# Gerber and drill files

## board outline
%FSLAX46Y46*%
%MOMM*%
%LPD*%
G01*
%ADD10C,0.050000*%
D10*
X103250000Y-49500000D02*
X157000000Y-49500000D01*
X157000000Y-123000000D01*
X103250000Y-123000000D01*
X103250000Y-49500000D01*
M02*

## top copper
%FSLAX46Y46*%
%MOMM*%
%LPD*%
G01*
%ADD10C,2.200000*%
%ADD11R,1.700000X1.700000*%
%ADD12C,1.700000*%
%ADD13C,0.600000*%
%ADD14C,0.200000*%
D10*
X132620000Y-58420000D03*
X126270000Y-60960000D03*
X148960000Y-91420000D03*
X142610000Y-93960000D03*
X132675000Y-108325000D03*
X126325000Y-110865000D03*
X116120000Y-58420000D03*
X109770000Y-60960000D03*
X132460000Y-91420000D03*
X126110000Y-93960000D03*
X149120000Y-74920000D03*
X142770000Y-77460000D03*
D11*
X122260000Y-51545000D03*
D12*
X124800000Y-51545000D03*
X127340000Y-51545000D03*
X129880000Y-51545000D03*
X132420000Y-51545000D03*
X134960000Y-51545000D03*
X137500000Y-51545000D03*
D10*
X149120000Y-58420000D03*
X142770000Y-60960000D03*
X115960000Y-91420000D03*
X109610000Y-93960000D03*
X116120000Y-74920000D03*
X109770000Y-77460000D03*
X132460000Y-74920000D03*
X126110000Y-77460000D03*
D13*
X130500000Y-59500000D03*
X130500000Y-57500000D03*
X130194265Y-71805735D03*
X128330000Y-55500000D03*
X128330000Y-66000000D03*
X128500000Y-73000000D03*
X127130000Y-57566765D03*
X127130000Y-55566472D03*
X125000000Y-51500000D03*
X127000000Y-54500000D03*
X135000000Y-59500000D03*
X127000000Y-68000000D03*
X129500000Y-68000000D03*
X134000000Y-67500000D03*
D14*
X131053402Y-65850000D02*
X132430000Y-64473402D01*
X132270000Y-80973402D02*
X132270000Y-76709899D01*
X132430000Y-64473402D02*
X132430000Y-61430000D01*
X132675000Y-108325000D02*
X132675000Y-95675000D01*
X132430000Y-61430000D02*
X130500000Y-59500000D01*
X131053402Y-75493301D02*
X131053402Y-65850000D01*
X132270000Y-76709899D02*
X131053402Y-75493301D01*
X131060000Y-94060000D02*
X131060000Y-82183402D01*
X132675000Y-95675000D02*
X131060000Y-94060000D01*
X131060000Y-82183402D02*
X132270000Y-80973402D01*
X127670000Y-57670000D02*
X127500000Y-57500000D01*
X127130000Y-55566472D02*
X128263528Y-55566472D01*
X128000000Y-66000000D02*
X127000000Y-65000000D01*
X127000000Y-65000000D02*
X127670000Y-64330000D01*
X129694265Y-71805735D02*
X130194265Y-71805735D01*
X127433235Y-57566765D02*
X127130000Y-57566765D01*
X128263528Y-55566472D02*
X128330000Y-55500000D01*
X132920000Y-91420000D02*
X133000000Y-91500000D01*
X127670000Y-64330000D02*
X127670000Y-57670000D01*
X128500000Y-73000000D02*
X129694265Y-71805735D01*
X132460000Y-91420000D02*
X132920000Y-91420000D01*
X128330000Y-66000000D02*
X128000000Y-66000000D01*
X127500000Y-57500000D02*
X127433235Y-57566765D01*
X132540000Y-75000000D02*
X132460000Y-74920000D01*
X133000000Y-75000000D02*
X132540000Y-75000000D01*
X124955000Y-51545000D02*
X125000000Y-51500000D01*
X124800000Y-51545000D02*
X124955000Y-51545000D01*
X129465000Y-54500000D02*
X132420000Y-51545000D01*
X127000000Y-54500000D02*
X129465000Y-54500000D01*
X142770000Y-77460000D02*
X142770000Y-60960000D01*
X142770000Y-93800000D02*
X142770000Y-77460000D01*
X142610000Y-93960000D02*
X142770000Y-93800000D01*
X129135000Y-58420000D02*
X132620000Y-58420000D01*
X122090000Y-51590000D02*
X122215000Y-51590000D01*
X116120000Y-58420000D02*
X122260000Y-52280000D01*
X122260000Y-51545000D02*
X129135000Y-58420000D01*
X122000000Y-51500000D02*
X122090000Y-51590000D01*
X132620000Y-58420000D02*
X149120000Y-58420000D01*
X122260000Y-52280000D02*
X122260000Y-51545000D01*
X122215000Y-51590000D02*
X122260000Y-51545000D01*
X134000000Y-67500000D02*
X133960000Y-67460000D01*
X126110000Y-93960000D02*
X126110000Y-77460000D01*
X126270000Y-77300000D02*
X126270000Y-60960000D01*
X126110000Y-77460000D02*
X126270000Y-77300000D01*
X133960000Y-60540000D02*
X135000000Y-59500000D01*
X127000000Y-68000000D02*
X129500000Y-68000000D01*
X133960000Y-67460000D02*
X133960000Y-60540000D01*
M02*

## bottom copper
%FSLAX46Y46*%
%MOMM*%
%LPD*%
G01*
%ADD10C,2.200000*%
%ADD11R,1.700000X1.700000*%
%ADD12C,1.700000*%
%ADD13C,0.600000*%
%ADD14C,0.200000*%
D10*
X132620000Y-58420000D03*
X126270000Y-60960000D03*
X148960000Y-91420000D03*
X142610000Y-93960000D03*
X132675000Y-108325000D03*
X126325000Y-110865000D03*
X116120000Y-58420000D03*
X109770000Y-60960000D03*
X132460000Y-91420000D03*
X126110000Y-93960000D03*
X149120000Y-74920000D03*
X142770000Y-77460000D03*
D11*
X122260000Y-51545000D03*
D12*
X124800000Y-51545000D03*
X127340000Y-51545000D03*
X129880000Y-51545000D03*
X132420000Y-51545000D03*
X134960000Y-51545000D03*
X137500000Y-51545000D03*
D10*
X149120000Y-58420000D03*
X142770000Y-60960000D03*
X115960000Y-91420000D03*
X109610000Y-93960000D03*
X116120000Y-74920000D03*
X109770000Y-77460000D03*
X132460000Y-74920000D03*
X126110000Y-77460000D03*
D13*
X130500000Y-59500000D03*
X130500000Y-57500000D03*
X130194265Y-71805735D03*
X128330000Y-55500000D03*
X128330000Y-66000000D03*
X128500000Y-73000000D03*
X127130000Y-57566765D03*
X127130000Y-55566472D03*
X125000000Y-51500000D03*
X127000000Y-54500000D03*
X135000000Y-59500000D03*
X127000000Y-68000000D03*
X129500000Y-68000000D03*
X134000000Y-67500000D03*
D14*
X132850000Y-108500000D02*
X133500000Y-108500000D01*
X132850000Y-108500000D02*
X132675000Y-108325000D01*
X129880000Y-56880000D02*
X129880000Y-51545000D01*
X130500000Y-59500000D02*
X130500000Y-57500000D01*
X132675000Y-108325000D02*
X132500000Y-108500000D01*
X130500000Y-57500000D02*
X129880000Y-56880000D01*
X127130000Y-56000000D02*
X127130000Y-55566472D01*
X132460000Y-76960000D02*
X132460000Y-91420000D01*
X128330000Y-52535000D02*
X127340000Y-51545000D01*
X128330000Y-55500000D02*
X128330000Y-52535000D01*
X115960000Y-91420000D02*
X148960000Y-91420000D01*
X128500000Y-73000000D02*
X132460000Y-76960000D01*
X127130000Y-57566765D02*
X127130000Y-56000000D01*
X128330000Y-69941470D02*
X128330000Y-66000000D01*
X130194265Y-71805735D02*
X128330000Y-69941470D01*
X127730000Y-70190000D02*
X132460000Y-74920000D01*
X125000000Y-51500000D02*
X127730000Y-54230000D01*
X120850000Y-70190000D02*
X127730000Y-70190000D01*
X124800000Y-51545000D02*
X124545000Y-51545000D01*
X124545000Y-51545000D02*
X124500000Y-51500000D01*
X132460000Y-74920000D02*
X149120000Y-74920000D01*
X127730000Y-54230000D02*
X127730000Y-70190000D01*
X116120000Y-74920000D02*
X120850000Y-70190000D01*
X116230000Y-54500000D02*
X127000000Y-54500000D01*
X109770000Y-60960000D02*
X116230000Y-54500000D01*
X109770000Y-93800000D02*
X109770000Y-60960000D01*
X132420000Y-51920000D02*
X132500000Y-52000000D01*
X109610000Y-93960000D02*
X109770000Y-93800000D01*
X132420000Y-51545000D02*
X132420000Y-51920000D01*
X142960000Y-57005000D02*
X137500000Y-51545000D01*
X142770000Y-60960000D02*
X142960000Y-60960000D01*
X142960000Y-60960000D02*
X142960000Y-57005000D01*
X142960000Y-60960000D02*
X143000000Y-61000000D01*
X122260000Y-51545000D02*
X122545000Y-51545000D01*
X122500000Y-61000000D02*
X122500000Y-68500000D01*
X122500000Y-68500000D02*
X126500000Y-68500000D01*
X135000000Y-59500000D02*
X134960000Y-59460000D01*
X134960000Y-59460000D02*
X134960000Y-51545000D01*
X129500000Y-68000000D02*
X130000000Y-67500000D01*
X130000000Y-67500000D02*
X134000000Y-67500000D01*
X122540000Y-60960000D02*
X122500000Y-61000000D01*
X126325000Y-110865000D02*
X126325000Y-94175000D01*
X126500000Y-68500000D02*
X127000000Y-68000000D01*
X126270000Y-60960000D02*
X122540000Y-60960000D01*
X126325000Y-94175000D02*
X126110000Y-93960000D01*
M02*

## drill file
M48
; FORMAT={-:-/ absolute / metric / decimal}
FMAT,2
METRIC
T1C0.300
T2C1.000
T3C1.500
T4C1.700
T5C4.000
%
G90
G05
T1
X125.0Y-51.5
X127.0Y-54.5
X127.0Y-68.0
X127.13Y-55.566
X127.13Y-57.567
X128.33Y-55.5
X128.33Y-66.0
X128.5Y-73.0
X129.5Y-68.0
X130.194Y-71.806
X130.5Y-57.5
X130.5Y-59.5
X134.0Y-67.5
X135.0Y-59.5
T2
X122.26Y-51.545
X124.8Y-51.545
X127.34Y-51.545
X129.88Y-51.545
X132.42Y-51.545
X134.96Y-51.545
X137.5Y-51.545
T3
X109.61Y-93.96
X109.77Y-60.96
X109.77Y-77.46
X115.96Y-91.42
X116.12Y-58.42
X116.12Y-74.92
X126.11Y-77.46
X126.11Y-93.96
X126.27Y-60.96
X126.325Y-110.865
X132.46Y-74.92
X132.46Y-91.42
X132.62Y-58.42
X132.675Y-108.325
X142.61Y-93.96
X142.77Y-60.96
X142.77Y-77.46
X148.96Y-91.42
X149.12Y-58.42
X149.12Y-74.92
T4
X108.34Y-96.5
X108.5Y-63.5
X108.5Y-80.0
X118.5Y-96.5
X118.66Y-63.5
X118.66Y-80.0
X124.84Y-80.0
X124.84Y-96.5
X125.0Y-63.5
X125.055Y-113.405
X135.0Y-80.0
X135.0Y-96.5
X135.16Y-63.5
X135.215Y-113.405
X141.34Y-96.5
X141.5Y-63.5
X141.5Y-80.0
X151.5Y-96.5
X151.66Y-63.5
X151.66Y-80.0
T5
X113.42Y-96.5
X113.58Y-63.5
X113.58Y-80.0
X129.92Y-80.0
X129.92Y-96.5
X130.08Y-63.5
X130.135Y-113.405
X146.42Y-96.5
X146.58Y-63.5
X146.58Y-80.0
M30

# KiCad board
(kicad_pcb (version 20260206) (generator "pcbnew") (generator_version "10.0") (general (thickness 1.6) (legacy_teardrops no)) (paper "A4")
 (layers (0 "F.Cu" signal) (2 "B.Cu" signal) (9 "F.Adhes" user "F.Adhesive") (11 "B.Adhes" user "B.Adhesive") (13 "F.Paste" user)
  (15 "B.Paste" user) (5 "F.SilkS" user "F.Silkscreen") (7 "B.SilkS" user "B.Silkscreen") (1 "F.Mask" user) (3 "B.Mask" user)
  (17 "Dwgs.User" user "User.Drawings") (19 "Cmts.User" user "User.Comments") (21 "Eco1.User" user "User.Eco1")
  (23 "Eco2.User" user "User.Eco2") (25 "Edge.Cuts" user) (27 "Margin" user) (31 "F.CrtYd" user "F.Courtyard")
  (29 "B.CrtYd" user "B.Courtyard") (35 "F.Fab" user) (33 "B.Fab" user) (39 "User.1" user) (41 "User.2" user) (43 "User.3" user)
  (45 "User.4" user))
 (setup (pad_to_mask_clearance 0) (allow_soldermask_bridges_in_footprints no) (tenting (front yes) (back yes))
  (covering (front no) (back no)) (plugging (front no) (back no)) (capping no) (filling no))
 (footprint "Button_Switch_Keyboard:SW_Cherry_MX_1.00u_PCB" (layer "F.Cu") (at 132.62 58.42)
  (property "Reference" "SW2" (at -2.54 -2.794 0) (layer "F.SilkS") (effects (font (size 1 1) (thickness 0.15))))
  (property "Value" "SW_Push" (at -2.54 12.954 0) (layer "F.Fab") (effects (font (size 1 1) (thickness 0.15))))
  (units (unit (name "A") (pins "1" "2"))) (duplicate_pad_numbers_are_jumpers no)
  (pad "" np_thru_hole circle (at -7.62 5.08) (size 1.7 1.7) (drill 1.7) (layers "*.Cu" "*.Mask"))
  (pad "" np_thru_hole circle (at -2.54 5.08) (size 4 4) (drill 4) (layers "*.Cu" "*.Mask"))
  (pad "" np_thru_hole circle (at 2.54 5.08) (size 1.7 1.7) (drill 1.7) (layers "*.Cu" "*.Mask"))
  (pad "1" thru_hole circle (at 0 0) (size 2.2 2.2) (drill 1.5) (layers "*.Cu" "*.Mask") (remove_unused_layers no) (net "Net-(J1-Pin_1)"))
  (pad "2" thru_hole circle (at -6.35 2.54) (size 2.2 2.2) (drill 1.5) (layers "*.Cu" "*.Mask") (remove_unused_layers no)
   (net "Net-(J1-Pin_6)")))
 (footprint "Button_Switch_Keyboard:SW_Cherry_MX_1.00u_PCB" (layer "F.Cu") (at 148.96 91.42)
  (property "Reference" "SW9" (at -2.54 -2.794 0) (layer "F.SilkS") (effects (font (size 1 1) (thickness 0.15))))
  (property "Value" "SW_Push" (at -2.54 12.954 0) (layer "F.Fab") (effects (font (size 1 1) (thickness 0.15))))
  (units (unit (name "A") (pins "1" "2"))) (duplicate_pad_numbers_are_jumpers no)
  (pad "" np_thru_hole circle (at -7.62 5.08) (size 1.7 1.7) (drill 1.7) (layers "*.Cu" "*.Mask"))
  (pad "" np_thru_hole circle (at -2.54 5.08) (size 4 4) (drill 4) (layers "*.Cu" "*.Mask"))
  (pad "" np_thru_hole circle (at 2.54 5.08) (size 1.7 1.7) (drill 1.7) (layers "*.Cu" "*.Mask"))
  (pad "1" thru_hole circle (at 0 0) (size 2.2 2.2) (drill 1.5) (layers "*.Cu" "*.Mask") (remove_unused_layers no) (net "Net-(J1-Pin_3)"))
  (pad "2" thru_hole circle (at -6.35 2.54) (size 2.2 2.2) (drill 1.5) (layers "*.Cu" "*.Mask") (remove_unused_layers no)
   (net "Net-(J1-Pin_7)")))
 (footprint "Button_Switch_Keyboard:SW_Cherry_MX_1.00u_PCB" (layer "F.Cu") (at 132.675 108.325)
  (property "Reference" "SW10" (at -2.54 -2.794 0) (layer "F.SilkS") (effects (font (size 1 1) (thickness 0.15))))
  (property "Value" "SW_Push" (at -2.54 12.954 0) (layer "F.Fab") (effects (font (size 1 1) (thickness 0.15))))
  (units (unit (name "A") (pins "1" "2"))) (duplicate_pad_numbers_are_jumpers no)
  (pad "" np_thru_hole circle (at -7.62 5.08) (size 1.7 1.7) (drill 1.7) (layers "*.Cu" "*.Mask"))
  (pad "" np_thru_hole circle (at -2.54 5.08) (size 4 4) (drill 4) (layers "*.Cu" "*.Mask"))
  (pad "" np_thru_hole circle (at 2.54 5.08) (size 1.7 1.7) (drill 1.7) (layers "*.Cu" "*.Mask"))
  (pad "1" thru_hole circle (at 0 0) (size 2.2 2.2) (drill 1.5) (layers "*.Cu" "*.Mask") (remove_unused_layers no) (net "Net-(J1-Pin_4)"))
  (pad "2" thru_hole circle (at -6.35 2.54) (size 2.2 2.2) (drill 1.5) (layers "*.Cu" "*.Mask") (remove_unused_layers no)
   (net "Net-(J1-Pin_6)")))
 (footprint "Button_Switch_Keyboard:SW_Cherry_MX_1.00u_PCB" (layer "F.Cu") (at 116.12 58.42)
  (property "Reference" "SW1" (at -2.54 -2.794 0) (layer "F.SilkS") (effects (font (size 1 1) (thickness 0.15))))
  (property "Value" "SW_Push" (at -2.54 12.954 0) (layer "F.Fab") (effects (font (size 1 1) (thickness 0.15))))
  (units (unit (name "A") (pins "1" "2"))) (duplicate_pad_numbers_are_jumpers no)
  (pad "" np_thru_hole circle (at -7.62 5.08) (size 1.7 1.7) (drill 1.7) (layers "*.Cu" "*.Mask"))
  (pad "" np_thru_hole circle (at -2.54 5.08) (size 4 4) (drill 4) (layers "*.Cu" "*.Mask"))
  (pad "" np_thru_hole circle (at 2.54 5.08) (size 1.7 1.7) (drill 1.7) (layers "*.Cu" "*.Mask"))
  (pad "1" thru_hole circle (at 0 0) (size 2.2 2.2) (drill 1.5) (layers "*.Cu" "*.Mask") (remove_unused_layers no) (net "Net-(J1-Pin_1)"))
  (pad "2" thru_hole circle (at -6.35 2.54) (size 2.2 2.2) (drill 1.5) (layers "*.Cu" "*.Mask") (remove_unused_layers no)
   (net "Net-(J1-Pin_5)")))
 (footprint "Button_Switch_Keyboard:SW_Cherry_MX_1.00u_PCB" (layer "F.Cu") (at 132.46 91.42)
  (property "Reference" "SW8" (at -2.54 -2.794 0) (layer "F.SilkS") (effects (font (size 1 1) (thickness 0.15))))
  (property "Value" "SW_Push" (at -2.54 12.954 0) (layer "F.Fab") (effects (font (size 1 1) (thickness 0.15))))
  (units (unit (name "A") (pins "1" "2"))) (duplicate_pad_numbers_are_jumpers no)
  (pad "" np_thru_hole circle (at -7.62 5.08) (size 1.7 1.7) (drill 1.7) (layers "*.Cu" "*.Mask"))
  (pad "" np_thru_hole circle (at -2.54 5.08) (size 4 4) (drill 4) (layers "*.Cu" "*.Mask"))
  (pad "" np_thru_hole circle (at 2.54 5.08) (size 1.7 1.7) (drill 1.7) (layers "*.Cu" "*.Mask"))
  (pad "1" thru_hole circle (at 0 0) (size 2.2 2.2) (drill 1.5) (layers "*.Cu" "*.Mask") (remove_unused_layers no) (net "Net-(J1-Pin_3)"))
  (pad "2" thru_hole circle (at -6.35 2.54) (size 2.2 2.2) (drill 1.5) (layers "*.Cu" "*.Mask") (remove_unused_layers no)
   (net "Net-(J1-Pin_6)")))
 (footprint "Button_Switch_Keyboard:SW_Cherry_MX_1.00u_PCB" (layer "F.Cu") (at 149.12 74.92)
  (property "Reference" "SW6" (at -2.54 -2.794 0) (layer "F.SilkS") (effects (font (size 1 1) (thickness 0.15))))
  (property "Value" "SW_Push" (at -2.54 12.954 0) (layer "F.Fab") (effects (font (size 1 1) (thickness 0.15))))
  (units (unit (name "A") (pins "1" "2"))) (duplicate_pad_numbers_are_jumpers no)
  (pad "" np_thru_hole circle (at -7.62 5.08) (size 1.7 1.7) (drill 1.7) (layers "*.Cu" "*.Mask"))
  (pad "" np_thru_hole circle (at -2.54 5.08) (size 4 4) (drill 4) (layers "*.Cu" "*.Mask"))
  (pad "" np_thru_hole circle (at 2.54 5.08) (size 1.7 1.7) (drill 1.7) (layers "*.Cu" "*.Mask"))
  (pad "1" thru_hole circle (at 0 0) (size 2.2 2.2) (drill 1.5) (layers "*.Cu" "*.Mask") (remove_unused_layers no) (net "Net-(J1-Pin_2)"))
  (pad "2" thru_hole circle (at -6.35 2.54) (size 2.2 2.2) (drill 1.5) (layers "*.Cu" "*.Mask") (remove_unused_layers no)
   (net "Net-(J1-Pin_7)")))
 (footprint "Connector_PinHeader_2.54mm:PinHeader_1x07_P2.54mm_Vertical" (layer "F.Cu") (at 122.26 51.545 90)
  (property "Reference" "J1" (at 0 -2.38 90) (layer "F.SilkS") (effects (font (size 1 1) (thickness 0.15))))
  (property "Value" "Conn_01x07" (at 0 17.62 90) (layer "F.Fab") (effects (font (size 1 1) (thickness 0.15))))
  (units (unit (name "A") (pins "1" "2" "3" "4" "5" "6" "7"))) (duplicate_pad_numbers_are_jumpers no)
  (pad "1" thru_hole rect (at 0 0 90) (size 1.7 1.7) (drill 1) (layers "*.Cu" "*.Mask") (remove_unused_layers no) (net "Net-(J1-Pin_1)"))
  (pad "2" thru_hole circle (at 0 2.54 90) (size 1.7 1.7) (drill 1) (layers "*.Cu" "*.Mask") (remove_unused_layers no)
   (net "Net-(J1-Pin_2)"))
  (pad "3" thru_hole circle (at 0 5.08 90) (size 1.7 1.7) (drill 1) (layers "*.Cu" "*.Mask") (remove_unused_layers no)
   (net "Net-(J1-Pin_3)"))
  (pad "4" thru_hole circle (at 0 7.62 90) (size 1.7 1.7) (drill 1) (layers "*.Cu" "*.Mask") (remove_unused_layers no)
   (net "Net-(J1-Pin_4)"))
  (pad "5" thru_hole circle (at 0 10.16 90) (size 1.7 1.7) (drill 1) (layers "*.Cu" "*.Mask") (remove_unused_layers no)
   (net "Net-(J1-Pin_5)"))
  (pad "6" thru_hole circle (at 0 12.7 90) (size 1.7 1.7) (drill 1) (layers "*.Cu" "*.Mask") (remove_unused_layers no)
   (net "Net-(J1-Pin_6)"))
  (pad "7" thru_hole circle (at 0 15.24 90) (size 1.7 1.7) (drill 1) (layers "*.Cu" "*.Mask") (remove_unused_layers no)
   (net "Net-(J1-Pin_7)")))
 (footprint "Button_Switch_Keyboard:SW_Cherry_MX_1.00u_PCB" (layer "F.Cu") (at 149.12 58.42)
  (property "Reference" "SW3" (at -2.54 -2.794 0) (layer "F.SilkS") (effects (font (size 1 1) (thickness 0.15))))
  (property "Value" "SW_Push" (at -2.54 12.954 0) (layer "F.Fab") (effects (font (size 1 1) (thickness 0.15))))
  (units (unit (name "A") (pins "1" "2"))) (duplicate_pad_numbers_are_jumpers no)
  (pad "" np_thru_hole circle (at -7.62 5.08) (size 1.7 1.7) (drill 1.7) (layers "*.Cu" "*.Mask"))
  (pad "" np_thru_hole circle (at -2.54 5.08) (size 4 4) (drill 4) (layers "*.Cu" "*.Mask"))
  (pad "" np_thru_hole circle (at 2.54 5.08) (size 1.7 1.7) (drill 1.7) (layers "*.Cu" "*.Mask"))
  (pad "1" thru_hole circle (at 0 0) (size 2.2 2.2) (drill 1.5) (layers "*.Cu" "*.Mask") (remove_unused_layers no) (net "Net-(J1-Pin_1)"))
  (pad "2" thru_hole circle (at -6.35 2.54) (size 2.2 2.2) (drill 1.5) (layers "*.Cu" "*.Mask") (remove_unused_layers no)
   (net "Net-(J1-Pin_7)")))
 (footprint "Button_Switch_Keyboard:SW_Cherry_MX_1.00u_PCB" (layer "F.Cu") (at 115.96 91.42)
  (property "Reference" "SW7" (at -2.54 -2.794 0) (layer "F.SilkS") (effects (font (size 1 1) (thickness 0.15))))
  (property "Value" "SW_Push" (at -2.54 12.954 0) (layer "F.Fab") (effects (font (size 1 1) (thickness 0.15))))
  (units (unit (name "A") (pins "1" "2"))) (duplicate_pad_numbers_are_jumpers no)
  (pad "" np_thru_hole circle (at -7.62 5.08) (size 1.7 1.7) (drill 1.7) (layers "*.Cu" "*.Mask"))
  (pad "" np_thru_hole circle (at -2.54 5.08) (size 4 4) (drill 4) (layers "*.Cu" "*.Mask"))
  (pad "" np_thru_hole circle (at 2.54 5.08) (size 1.7 1.7) (drill 1.7) (layers "*.Cu" "*.Mask"))
  (pad "1" thru_hole circle (at 0 0) (size 2.2 2.2) (drill 1.5) (layers "*.Cu" "*.Mask") (remove_unused_layers no) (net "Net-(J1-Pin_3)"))
  (pad "2" thru_hole circle (at -6.35 2.54) (size 2.2 2.2) (drill 1.5) (layers "*.Cu" "*.Mask") (remove_unused_layers no)
   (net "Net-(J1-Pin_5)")))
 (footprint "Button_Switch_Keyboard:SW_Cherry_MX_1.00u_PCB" (layer "F.Cu") (at 116.12 74.92)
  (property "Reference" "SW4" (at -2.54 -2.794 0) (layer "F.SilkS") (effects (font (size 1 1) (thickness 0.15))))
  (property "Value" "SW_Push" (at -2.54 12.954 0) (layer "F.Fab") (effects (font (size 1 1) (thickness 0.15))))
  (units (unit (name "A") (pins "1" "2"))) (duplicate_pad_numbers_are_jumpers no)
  (pad "" np_thru_hole circle (at -7.62 5.08) (size 1.7 1.7) (drill 1.7) (layers "*.Cu" "*.Mask"))
  (pad "" np_thru_hole circle (at -2.54 5.08) (size 4 4) (drill 4) (layers "*.Cu" "*.Mask"))
  (pad "" np_thru_hole circle (at 2.54 5.08) (size 1.7 1.7) (drill 1.7) (layers "*.Cu" "*.Mask"))
  (pad "1" thru_hole circle (at 0 0) (size 2.2 2.2) (drill 1.5) (layers "*.Cu" "*.Mask") (remove_unused_layers no) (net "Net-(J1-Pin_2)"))
  (pad "2" thru_hole circle (at -6.35 2.54) (size 2.2 2.2) (drill 1.5) (layers "*.Cu" "*.Mask") (remove_unused_layers no)
   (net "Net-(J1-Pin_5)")))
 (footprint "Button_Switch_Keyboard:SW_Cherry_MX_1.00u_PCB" (layer "F.Cu") (at 132.46 74.92)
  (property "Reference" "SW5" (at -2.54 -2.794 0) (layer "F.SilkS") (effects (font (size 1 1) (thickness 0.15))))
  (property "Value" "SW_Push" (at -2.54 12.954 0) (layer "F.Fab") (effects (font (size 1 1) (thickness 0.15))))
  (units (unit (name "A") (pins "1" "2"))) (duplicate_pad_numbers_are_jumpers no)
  (pad "" np_thru_hole circle (at -7.62 5.08) (size 1.7 1.7) (drill 1.7) (layers "*.Cu" "*.Mask"))
  (pad "" np_thru_hole circle (at -2.54 5.08) (size 4 4) (drill 4) (layers "*.Cu" "*.Mask"))
  (pad "" np_thru_hole circle (at 2.54 5.08) (size 1.7 1.7) (drill 1.7) (layers "*.Cu" "*.Mask"))
  (pad "1" thru_hole circle (at 0 0) (size 2.2 2.2) (drill 1.5) (layers "*.Cu" "*.Mask") (remove_unused_layers no) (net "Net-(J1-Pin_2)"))
  (pad "2" thru_hole circle (at -6.35 2.54) (size 2.2 2.2) (drill 1.5) (layers "*.Cu" "*.Mask") (remove_unused_layers no)
   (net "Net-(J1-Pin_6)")))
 (gr_rect (start 103.25 49.5) (end 157 123) (stroke (width 0.05) (type default)) (fill no) (layer "Edge.Cuts"))
 (segment (start 131.053402 65.85) (end 132.43 64.473402) (width 0.2) (layer "F.Cu") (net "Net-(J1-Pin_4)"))
 (segment (start 132.27 80.973402) (end 132.27 76.709899) (width 0.2) (layer "F.Cu") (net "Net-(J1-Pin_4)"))
 (segment (start 132.43 64.473402) (end 132.43 61.43) (width 0.2) (layer "F.Cu") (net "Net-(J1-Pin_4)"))
 (segment (start 132.675 108.325) (end 132.675 95.675) (width 0.2) (layer "F.Cu") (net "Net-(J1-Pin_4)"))
 (segment (start 132.43 61.43) (end 130.5 59.5) (width 0.2) (layer "F.Cu") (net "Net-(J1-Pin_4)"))
 (segment (start 131.053402 75.493301) (end 131.053402 65.85) (width 0.2) (layer "F.Cu") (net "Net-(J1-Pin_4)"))
 (segment (start 132.27 76.709899) (end 131.053402 75.493301) (width 0.2) (layer "F.Cu") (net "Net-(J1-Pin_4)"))
 (segment (start 131.06 94.06) (end 131.06 82.183402) (width 0.2) (layer "F.Cu") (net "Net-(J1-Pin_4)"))
 (segment (start 132.675 95.675) (end 131.06 94.06) (width 0.2) (layer "F.Cu") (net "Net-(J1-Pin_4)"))
 (segment (start 131.06 82.183402) (end 132.27 80.973402) (width 0.2) (layer "F.Cu") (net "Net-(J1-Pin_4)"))
 (via (at 130.5 59.5) (size 0.6) (drill 0.3) (layers "F.Cu" "B.Cu") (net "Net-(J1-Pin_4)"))
 (via (at 130.5 57.5) (size 0.6) (drill 0.3) (layers "F.Cu" "B.Cu") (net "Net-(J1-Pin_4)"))
 (segment (start 132.85 108.5) (end 133.5 108.5) (width 0.2) (layer "B.Cu") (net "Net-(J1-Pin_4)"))
 (segment (start 132.85 108.5) (end 132.675 108.325) (width 0.2) (layer "B.Cu") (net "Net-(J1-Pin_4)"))
 (segment (start 129.88 56.88) (end 129.88 51.545) (width 0.2) (layer "B.Cu") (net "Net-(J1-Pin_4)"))
 (segment (start 130.5 59.5) (end 130.5 57.5) (width 0.2) (layer "B.Cu") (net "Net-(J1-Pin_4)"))
 (segment (start 132.675 108.325) (end 132.5 108.5) (width 0.2) (layer "B.Cu") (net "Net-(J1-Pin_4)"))
 (segment (start 130.5 57.5) (end 129.88 56.88) (width 0.2) (layer "B.Cu") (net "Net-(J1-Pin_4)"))
 (segment (start 127.67 57.67) (end 127.5 57.5) (width 0.2) (layer "F.Cu") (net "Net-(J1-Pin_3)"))
 (segment (start 127.13 55.566472) (end 128.263528 55.566472) (width 0.2) (layer "F.Cu") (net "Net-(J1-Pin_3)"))
 (segment (start 128 66) (end 127 65) (width 0.2) (layer "F.Cu") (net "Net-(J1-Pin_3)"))
 (segment (start 127 65) (end 127.67 64.33) (width 0.2) (layer "F.Cu") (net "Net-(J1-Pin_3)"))
 (segment (start 129.694265 71.805735) (end 130.194265 71.805735) (width 0.2) (layer "F.Cu") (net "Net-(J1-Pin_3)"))
 (segment (start 127.433235 57.566765) (end 127.13 57.566765) (width 0.2) (layer "F.Cu") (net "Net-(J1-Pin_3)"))
 (segment (start 128.263528 55.566472) (end 128.33 55.5) (width 0.2) (layer "F.Cu") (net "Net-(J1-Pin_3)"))
 (segment (start 132.92 91.42) (end 133 91.5) (width 0.2) (layer "F.Cu") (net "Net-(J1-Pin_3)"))
 (segment (start 127.67 64.33) (end 127.67 57.67) (width 0.2) (layer "F.Cu") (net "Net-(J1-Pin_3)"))
 (segment (start 128.5 73) (end 129.694265 71.805735) (width 0.2) (layer "F.Cu") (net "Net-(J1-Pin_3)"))
 (segment (start 132.46 91.42) (end 132.92 91.42) (width 0.2) (layer "F.Cu") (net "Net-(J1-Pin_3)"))
 (segment (start 128.33 66) (end 128 66) (width 0.2) (layer "F.Cu") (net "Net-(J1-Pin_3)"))
 (segment (start 127.5 57.5) (end 127.433235 57.566765) (width 0.2) (layer "F.Cu") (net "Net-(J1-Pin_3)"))
 (via (at 130.194265 71.805735) (size 0.6) (drill 0.3) (layers "F.Cu" "B.Cu") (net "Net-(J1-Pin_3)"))
 (via (at 128.33 55.5) (size 0.6) (drill 0.3) (layers "F.Cu" "B.Cu") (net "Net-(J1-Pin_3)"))
 (via (at 128.33 66) (size 0.6) (drill 0.3) (layers "F.Cu" "B.Cu") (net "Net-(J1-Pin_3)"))
 (via (at 128.5 73) (size 0.6) (drill 0.3) (layers "F.Cu" "B.Cu") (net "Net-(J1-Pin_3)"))
 (via (at 127.13 57.566765) (size 0.6) (drill 0.3) (layers "F.Cu" "B.Cu") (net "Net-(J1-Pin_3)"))
 (via (at 127.13 55.566472) (size 0.6) (drill 0.3) (layers "F.Cu" "B.Cu") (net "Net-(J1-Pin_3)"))
 (segment (start 127.13 56) (end 127.13 55.566472) (width 0.2) (layer "B.Cu") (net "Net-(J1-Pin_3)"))
 (segment (start 132.46 76.96) (end 132.46 91.42) (width 0.2) (layer "B.Cu") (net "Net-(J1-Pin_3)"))
 (segment (start 128.33 52.535) (end 127.34 51.545) (width 0.2) (layer "B.Cu") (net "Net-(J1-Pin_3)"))
 (segment (start 128.33 55.5) (end 128.33 52.535) (width 0.2) (layer "B.Cu") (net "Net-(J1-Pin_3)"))
 (segment (start 115.96 91.42) (end 148.96 91.42) (width 0.2) (layer "B.Cu") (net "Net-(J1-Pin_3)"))
 (segment (start 128.5 73) (end 132.46 76.96) (width 0.2) (layer "B.Cu") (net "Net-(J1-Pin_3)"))
 (segment (start 127.13 57.566765) (end 127.13 56) (width 0.2) (layer "B.Cu") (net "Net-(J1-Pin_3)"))
 (segment (start 128.33 69.94147) (end 128.33 66) (width 0.2) (layer "B.Cu") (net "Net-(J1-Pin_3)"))
 (segment (start 130.194265 71.805735) (end 128.33 69.94147) (width 0.2) (layer "B.Cu") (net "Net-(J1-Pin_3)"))
 (segment (start 132.54 75) (end 132.46 74.92) (width 0.2) (layer "F.Cu") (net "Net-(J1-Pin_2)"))
 (segment (start 133 75) (end 132.54 75) (width 0.2) (layer "F.Cu") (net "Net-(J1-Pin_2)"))
 (segment (start 124.955 51.545) (end 125 51.5) (width 0.2) (layer "F.Cu") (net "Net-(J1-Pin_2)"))
 (segment (start 124.8 51.545) (end 124.955 51.545) (width 0.2) (layer "F.Cu") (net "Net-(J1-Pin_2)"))
 (via (at 125 51.5) (size 0.6) (drill 0.3) (layers "F.Cu" "B.Cu") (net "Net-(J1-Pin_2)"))
 (segment (start 127.73 70.19) (end 132.46 74.92) (width 0.2) (layer "B.Cu") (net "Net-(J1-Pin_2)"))
 (segment (start 125 51.5) (end 127.73 54.23) (width 0.2) (layer "B.Cu") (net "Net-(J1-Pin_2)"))
 (segment (start 120.85 70.19) (end 127.73 70.19) (width 0.2) (layer "B.Cu") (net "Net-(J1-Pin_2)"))
 (segment (start 124.8 51.545) (end 124.545 51.545) (width 0.2) (layer "B.Cu") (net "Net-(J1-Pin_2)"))
 (segment (start 124.545 51.545) (end 124.5 51.5) (width 0.2) (layer "B.Cu") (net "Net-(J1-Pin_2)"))
 (segment (start 132.46 74.92) (end 149.12 74.92) (width 0.2) (layer "B.Cu") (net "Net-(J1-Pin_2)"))
 (segment (start 127.73 54.23) (end 127.73 70.19) (width 0.2) (layer "B.Cu") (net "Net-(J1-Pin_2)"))
 (segment (start 116.12 74.92) (end 120.85 70.19) (width 0.2) (layer "B.Cu") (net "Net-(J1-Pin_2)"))
 (segment (start 129.465 54.5) (end 132.42 51.545) (width 0.2) (layer "F.Cu") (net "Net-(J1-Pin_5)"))
 (segment (start 127 54.5) (end 129.465 54.5) (width 0.2) (layer "F.Cu") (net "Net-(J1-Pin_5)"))
 (via (at 127 54.5) (size 0.6) (drill 0.3) (layers "F.Cu" "B.Cu") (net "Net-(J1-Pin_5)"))
 (segment (start 116.23 54.5) (end 127 54.5) (width 0.2) (layer "B.Cu") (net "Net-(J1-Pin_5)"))
 (segment (start 109.77 60.96) (end 116.23 54.5) (width 0.2) (layer "B.Cu") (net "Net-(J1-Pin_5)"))
 (segment (start 109.77 93.8) (end 109.77 60.96) (width 0.2) (layer "B.Cu") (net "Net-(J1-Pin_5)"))
 (segment (start 132.42 51.92) (end 132.5 52) (width 0.2) (layer "B.Cu") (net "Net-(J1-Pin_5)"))
 (segment (start 109.61 93.96) (end 109.77 93.8) (width 0.2) (layer "B.Cu") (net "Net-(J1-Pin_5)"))
 (segment (start 132.42 51.545) (end 132.42 51.92) (width 0.2) (layer "B.Cu") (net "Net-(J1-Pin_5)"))
 (segment (start 142.77 77.46) (end 142.77 60.96) (width 0.2) (layer "F.Cu") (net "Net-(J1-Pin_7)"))
 (segment (start 142.77 93.8) (end 142.77 77.46) (width 0.2) (layer "F.Cu") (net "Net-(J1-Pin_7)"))
 (segment (start 142.61 93.96) (end 142.77 93.8) (width 0.2) (layer "F.Cu") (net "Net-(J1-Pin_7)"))
 (segment (start 142.96 57.005) (end 137.5 51.545) (width 0.2) (layer "B.Cu") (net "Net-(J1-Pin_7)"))
 (segment (start 142.77 60.96) (end 142.96 60.96) (width 0.2) (layer "B.Cu") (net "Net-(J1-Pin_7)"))
 (segment (start 142.96 60.96) (end 142.96 57.005) (width 0.2) (layer "B.Cu") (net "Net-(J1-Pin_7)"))
 (segment (start 142.96 60.96) (end 143 61) (width 0.2) (layer "B.Cu") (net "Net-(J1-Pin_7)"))
 (segment (start 129.135 58.42) (end 132.62 58.42) (width 0.2) (layer "F.Cu") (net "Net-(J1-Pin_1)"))
 (segment (start 122.09 51.59) (end 122.215 51.59) (width 0.2) (layer "F.Cu") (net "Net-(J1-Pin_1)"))
 (segment (start 116.12 58.42) (end 122.26 52.28) (width 0.2) (layer "F.Cu") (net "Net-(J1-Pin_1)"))
 (segment (start 122.26 51.545) (end 129.135 58.42) (width 0.2) (layer "F.Cu") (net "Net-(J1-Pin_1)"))
 (segment (start 122 51.5) (end 122.09 51.59) (width 0.2) (layer "F.Cu") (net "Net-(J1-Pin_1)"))
 (segment (start 132.62 58.42) (end 149.12 58.42) (width 0.2) (layer "F.Cu") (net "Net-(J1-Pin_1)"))
 (segment (start 122.26 52.28) (end 122.26 51.545) (width 0.2) (layer "F.Cu") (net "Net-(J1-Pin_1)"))
 (segment (start 122.215 51.59) (end 122.26 51.545) (width 0.2) (layer "F.Cu") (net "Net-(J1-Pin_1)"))
 (segment (start 122.26 51.545) (end 122.545 51.545) (width 0.2) (layer "B.Cu") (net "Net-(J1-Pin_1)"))
 (segment (start 134 67.5) (end 133.96 67.46) (width 0.2) (layer "F.Cu") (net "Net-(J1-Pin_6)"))
 (segment (start 126.11 93.96) (end 126.11 77.46) (width 0.2) (layer "F.Cu") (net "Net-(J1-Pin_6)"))
 (segment (start 126.27 77.3) (end 126.27 60.96) (width 0.2) (layer "F.Cu") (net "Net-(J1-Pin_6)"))
 (segment (start 126.11 77.46) (end 126.27 77.3) (width 0.2) (layer "F.Cu") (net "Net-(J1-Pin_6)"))
 (segment (start 133.96 60.54) (end 135 59.5) (width 0.2) (layer "F.Cu") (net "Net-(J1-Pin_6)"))
 (segment (start 127 68) (end 129.5 68) (width 0.2) (layer "F.Cu") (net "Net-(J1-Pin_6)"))
 (segment (start 133.96 67.46) (end 133.96 60.54) (width 0.2) (layer "F.Cu") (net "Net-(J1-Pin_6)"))
 (via (at 135 59.5) (size 0.6) (drill 0.3) (layers "F.Cu" "B.Cu") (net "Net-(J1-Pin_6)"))
 (via (at 127 68) (size 0.6) (drill 0.3) (layers "F.Cu" "B.Cu") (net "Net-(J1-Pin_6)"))
 (via (at 129.5 68) (size 0.6) (drill 0.3) (layers "F.Cu" "B.Cu") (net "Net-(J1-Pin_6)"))
 (via (at 134 67.5) (size 0.6) (drill 0.3) (layers "F.Cu" "B.Cu") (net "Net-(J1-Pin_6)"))
 (segment (start 122.5 61) (end 122.5 68.5) (width 0.2) (layer "B.Cu") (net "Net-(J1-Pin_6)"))
 (segment (start 122.5 68.5) (end 126.5 68.5) (width 0.2) (layer "B.Cu") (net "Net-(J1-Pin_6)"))
 (segment (start 135 59.5) (end 134.96 59.46) (width 0.2) (layer "B.Cu") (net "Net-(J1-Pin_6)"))
 (segment (start 134.96 59.46) (end 134.96 51.545) (width 0.2) (layer "B.Cu") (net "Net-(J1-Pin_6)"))
 (segment (start 129.5 68) (end 130 67.5) (width 0.2) (layer "B.Cu") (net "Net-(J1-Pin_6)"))
 (segment (start 130 67.5) (end 134 67.5) (width 0.2) (layer "B.Cu") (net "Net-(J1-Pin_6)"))
 (segment (start 122.54 60.96) (end 122.5 61) (width 0.2) (layer "B.Cu") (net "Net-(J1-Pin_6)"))
 (segment (start 126.325 110.865) (end 126.325 94.175) (width 0.2) (layer "B.Cu") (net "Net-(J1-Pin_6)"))
 (segment (start 126.5 68.5) (end 127 68) (width 0.2) (layer "B.Cu") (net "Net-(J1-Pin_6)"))
 (segment (start 126.27 60.96) (end 122.54 60.96) (width 0.2) (layer "B.Cu") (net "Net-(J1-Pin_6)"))
 (segment (start 126.325 94.175) (end 126.11 93.96) (width 0.2) (layer "B.Cu") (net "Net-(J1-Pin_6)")))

